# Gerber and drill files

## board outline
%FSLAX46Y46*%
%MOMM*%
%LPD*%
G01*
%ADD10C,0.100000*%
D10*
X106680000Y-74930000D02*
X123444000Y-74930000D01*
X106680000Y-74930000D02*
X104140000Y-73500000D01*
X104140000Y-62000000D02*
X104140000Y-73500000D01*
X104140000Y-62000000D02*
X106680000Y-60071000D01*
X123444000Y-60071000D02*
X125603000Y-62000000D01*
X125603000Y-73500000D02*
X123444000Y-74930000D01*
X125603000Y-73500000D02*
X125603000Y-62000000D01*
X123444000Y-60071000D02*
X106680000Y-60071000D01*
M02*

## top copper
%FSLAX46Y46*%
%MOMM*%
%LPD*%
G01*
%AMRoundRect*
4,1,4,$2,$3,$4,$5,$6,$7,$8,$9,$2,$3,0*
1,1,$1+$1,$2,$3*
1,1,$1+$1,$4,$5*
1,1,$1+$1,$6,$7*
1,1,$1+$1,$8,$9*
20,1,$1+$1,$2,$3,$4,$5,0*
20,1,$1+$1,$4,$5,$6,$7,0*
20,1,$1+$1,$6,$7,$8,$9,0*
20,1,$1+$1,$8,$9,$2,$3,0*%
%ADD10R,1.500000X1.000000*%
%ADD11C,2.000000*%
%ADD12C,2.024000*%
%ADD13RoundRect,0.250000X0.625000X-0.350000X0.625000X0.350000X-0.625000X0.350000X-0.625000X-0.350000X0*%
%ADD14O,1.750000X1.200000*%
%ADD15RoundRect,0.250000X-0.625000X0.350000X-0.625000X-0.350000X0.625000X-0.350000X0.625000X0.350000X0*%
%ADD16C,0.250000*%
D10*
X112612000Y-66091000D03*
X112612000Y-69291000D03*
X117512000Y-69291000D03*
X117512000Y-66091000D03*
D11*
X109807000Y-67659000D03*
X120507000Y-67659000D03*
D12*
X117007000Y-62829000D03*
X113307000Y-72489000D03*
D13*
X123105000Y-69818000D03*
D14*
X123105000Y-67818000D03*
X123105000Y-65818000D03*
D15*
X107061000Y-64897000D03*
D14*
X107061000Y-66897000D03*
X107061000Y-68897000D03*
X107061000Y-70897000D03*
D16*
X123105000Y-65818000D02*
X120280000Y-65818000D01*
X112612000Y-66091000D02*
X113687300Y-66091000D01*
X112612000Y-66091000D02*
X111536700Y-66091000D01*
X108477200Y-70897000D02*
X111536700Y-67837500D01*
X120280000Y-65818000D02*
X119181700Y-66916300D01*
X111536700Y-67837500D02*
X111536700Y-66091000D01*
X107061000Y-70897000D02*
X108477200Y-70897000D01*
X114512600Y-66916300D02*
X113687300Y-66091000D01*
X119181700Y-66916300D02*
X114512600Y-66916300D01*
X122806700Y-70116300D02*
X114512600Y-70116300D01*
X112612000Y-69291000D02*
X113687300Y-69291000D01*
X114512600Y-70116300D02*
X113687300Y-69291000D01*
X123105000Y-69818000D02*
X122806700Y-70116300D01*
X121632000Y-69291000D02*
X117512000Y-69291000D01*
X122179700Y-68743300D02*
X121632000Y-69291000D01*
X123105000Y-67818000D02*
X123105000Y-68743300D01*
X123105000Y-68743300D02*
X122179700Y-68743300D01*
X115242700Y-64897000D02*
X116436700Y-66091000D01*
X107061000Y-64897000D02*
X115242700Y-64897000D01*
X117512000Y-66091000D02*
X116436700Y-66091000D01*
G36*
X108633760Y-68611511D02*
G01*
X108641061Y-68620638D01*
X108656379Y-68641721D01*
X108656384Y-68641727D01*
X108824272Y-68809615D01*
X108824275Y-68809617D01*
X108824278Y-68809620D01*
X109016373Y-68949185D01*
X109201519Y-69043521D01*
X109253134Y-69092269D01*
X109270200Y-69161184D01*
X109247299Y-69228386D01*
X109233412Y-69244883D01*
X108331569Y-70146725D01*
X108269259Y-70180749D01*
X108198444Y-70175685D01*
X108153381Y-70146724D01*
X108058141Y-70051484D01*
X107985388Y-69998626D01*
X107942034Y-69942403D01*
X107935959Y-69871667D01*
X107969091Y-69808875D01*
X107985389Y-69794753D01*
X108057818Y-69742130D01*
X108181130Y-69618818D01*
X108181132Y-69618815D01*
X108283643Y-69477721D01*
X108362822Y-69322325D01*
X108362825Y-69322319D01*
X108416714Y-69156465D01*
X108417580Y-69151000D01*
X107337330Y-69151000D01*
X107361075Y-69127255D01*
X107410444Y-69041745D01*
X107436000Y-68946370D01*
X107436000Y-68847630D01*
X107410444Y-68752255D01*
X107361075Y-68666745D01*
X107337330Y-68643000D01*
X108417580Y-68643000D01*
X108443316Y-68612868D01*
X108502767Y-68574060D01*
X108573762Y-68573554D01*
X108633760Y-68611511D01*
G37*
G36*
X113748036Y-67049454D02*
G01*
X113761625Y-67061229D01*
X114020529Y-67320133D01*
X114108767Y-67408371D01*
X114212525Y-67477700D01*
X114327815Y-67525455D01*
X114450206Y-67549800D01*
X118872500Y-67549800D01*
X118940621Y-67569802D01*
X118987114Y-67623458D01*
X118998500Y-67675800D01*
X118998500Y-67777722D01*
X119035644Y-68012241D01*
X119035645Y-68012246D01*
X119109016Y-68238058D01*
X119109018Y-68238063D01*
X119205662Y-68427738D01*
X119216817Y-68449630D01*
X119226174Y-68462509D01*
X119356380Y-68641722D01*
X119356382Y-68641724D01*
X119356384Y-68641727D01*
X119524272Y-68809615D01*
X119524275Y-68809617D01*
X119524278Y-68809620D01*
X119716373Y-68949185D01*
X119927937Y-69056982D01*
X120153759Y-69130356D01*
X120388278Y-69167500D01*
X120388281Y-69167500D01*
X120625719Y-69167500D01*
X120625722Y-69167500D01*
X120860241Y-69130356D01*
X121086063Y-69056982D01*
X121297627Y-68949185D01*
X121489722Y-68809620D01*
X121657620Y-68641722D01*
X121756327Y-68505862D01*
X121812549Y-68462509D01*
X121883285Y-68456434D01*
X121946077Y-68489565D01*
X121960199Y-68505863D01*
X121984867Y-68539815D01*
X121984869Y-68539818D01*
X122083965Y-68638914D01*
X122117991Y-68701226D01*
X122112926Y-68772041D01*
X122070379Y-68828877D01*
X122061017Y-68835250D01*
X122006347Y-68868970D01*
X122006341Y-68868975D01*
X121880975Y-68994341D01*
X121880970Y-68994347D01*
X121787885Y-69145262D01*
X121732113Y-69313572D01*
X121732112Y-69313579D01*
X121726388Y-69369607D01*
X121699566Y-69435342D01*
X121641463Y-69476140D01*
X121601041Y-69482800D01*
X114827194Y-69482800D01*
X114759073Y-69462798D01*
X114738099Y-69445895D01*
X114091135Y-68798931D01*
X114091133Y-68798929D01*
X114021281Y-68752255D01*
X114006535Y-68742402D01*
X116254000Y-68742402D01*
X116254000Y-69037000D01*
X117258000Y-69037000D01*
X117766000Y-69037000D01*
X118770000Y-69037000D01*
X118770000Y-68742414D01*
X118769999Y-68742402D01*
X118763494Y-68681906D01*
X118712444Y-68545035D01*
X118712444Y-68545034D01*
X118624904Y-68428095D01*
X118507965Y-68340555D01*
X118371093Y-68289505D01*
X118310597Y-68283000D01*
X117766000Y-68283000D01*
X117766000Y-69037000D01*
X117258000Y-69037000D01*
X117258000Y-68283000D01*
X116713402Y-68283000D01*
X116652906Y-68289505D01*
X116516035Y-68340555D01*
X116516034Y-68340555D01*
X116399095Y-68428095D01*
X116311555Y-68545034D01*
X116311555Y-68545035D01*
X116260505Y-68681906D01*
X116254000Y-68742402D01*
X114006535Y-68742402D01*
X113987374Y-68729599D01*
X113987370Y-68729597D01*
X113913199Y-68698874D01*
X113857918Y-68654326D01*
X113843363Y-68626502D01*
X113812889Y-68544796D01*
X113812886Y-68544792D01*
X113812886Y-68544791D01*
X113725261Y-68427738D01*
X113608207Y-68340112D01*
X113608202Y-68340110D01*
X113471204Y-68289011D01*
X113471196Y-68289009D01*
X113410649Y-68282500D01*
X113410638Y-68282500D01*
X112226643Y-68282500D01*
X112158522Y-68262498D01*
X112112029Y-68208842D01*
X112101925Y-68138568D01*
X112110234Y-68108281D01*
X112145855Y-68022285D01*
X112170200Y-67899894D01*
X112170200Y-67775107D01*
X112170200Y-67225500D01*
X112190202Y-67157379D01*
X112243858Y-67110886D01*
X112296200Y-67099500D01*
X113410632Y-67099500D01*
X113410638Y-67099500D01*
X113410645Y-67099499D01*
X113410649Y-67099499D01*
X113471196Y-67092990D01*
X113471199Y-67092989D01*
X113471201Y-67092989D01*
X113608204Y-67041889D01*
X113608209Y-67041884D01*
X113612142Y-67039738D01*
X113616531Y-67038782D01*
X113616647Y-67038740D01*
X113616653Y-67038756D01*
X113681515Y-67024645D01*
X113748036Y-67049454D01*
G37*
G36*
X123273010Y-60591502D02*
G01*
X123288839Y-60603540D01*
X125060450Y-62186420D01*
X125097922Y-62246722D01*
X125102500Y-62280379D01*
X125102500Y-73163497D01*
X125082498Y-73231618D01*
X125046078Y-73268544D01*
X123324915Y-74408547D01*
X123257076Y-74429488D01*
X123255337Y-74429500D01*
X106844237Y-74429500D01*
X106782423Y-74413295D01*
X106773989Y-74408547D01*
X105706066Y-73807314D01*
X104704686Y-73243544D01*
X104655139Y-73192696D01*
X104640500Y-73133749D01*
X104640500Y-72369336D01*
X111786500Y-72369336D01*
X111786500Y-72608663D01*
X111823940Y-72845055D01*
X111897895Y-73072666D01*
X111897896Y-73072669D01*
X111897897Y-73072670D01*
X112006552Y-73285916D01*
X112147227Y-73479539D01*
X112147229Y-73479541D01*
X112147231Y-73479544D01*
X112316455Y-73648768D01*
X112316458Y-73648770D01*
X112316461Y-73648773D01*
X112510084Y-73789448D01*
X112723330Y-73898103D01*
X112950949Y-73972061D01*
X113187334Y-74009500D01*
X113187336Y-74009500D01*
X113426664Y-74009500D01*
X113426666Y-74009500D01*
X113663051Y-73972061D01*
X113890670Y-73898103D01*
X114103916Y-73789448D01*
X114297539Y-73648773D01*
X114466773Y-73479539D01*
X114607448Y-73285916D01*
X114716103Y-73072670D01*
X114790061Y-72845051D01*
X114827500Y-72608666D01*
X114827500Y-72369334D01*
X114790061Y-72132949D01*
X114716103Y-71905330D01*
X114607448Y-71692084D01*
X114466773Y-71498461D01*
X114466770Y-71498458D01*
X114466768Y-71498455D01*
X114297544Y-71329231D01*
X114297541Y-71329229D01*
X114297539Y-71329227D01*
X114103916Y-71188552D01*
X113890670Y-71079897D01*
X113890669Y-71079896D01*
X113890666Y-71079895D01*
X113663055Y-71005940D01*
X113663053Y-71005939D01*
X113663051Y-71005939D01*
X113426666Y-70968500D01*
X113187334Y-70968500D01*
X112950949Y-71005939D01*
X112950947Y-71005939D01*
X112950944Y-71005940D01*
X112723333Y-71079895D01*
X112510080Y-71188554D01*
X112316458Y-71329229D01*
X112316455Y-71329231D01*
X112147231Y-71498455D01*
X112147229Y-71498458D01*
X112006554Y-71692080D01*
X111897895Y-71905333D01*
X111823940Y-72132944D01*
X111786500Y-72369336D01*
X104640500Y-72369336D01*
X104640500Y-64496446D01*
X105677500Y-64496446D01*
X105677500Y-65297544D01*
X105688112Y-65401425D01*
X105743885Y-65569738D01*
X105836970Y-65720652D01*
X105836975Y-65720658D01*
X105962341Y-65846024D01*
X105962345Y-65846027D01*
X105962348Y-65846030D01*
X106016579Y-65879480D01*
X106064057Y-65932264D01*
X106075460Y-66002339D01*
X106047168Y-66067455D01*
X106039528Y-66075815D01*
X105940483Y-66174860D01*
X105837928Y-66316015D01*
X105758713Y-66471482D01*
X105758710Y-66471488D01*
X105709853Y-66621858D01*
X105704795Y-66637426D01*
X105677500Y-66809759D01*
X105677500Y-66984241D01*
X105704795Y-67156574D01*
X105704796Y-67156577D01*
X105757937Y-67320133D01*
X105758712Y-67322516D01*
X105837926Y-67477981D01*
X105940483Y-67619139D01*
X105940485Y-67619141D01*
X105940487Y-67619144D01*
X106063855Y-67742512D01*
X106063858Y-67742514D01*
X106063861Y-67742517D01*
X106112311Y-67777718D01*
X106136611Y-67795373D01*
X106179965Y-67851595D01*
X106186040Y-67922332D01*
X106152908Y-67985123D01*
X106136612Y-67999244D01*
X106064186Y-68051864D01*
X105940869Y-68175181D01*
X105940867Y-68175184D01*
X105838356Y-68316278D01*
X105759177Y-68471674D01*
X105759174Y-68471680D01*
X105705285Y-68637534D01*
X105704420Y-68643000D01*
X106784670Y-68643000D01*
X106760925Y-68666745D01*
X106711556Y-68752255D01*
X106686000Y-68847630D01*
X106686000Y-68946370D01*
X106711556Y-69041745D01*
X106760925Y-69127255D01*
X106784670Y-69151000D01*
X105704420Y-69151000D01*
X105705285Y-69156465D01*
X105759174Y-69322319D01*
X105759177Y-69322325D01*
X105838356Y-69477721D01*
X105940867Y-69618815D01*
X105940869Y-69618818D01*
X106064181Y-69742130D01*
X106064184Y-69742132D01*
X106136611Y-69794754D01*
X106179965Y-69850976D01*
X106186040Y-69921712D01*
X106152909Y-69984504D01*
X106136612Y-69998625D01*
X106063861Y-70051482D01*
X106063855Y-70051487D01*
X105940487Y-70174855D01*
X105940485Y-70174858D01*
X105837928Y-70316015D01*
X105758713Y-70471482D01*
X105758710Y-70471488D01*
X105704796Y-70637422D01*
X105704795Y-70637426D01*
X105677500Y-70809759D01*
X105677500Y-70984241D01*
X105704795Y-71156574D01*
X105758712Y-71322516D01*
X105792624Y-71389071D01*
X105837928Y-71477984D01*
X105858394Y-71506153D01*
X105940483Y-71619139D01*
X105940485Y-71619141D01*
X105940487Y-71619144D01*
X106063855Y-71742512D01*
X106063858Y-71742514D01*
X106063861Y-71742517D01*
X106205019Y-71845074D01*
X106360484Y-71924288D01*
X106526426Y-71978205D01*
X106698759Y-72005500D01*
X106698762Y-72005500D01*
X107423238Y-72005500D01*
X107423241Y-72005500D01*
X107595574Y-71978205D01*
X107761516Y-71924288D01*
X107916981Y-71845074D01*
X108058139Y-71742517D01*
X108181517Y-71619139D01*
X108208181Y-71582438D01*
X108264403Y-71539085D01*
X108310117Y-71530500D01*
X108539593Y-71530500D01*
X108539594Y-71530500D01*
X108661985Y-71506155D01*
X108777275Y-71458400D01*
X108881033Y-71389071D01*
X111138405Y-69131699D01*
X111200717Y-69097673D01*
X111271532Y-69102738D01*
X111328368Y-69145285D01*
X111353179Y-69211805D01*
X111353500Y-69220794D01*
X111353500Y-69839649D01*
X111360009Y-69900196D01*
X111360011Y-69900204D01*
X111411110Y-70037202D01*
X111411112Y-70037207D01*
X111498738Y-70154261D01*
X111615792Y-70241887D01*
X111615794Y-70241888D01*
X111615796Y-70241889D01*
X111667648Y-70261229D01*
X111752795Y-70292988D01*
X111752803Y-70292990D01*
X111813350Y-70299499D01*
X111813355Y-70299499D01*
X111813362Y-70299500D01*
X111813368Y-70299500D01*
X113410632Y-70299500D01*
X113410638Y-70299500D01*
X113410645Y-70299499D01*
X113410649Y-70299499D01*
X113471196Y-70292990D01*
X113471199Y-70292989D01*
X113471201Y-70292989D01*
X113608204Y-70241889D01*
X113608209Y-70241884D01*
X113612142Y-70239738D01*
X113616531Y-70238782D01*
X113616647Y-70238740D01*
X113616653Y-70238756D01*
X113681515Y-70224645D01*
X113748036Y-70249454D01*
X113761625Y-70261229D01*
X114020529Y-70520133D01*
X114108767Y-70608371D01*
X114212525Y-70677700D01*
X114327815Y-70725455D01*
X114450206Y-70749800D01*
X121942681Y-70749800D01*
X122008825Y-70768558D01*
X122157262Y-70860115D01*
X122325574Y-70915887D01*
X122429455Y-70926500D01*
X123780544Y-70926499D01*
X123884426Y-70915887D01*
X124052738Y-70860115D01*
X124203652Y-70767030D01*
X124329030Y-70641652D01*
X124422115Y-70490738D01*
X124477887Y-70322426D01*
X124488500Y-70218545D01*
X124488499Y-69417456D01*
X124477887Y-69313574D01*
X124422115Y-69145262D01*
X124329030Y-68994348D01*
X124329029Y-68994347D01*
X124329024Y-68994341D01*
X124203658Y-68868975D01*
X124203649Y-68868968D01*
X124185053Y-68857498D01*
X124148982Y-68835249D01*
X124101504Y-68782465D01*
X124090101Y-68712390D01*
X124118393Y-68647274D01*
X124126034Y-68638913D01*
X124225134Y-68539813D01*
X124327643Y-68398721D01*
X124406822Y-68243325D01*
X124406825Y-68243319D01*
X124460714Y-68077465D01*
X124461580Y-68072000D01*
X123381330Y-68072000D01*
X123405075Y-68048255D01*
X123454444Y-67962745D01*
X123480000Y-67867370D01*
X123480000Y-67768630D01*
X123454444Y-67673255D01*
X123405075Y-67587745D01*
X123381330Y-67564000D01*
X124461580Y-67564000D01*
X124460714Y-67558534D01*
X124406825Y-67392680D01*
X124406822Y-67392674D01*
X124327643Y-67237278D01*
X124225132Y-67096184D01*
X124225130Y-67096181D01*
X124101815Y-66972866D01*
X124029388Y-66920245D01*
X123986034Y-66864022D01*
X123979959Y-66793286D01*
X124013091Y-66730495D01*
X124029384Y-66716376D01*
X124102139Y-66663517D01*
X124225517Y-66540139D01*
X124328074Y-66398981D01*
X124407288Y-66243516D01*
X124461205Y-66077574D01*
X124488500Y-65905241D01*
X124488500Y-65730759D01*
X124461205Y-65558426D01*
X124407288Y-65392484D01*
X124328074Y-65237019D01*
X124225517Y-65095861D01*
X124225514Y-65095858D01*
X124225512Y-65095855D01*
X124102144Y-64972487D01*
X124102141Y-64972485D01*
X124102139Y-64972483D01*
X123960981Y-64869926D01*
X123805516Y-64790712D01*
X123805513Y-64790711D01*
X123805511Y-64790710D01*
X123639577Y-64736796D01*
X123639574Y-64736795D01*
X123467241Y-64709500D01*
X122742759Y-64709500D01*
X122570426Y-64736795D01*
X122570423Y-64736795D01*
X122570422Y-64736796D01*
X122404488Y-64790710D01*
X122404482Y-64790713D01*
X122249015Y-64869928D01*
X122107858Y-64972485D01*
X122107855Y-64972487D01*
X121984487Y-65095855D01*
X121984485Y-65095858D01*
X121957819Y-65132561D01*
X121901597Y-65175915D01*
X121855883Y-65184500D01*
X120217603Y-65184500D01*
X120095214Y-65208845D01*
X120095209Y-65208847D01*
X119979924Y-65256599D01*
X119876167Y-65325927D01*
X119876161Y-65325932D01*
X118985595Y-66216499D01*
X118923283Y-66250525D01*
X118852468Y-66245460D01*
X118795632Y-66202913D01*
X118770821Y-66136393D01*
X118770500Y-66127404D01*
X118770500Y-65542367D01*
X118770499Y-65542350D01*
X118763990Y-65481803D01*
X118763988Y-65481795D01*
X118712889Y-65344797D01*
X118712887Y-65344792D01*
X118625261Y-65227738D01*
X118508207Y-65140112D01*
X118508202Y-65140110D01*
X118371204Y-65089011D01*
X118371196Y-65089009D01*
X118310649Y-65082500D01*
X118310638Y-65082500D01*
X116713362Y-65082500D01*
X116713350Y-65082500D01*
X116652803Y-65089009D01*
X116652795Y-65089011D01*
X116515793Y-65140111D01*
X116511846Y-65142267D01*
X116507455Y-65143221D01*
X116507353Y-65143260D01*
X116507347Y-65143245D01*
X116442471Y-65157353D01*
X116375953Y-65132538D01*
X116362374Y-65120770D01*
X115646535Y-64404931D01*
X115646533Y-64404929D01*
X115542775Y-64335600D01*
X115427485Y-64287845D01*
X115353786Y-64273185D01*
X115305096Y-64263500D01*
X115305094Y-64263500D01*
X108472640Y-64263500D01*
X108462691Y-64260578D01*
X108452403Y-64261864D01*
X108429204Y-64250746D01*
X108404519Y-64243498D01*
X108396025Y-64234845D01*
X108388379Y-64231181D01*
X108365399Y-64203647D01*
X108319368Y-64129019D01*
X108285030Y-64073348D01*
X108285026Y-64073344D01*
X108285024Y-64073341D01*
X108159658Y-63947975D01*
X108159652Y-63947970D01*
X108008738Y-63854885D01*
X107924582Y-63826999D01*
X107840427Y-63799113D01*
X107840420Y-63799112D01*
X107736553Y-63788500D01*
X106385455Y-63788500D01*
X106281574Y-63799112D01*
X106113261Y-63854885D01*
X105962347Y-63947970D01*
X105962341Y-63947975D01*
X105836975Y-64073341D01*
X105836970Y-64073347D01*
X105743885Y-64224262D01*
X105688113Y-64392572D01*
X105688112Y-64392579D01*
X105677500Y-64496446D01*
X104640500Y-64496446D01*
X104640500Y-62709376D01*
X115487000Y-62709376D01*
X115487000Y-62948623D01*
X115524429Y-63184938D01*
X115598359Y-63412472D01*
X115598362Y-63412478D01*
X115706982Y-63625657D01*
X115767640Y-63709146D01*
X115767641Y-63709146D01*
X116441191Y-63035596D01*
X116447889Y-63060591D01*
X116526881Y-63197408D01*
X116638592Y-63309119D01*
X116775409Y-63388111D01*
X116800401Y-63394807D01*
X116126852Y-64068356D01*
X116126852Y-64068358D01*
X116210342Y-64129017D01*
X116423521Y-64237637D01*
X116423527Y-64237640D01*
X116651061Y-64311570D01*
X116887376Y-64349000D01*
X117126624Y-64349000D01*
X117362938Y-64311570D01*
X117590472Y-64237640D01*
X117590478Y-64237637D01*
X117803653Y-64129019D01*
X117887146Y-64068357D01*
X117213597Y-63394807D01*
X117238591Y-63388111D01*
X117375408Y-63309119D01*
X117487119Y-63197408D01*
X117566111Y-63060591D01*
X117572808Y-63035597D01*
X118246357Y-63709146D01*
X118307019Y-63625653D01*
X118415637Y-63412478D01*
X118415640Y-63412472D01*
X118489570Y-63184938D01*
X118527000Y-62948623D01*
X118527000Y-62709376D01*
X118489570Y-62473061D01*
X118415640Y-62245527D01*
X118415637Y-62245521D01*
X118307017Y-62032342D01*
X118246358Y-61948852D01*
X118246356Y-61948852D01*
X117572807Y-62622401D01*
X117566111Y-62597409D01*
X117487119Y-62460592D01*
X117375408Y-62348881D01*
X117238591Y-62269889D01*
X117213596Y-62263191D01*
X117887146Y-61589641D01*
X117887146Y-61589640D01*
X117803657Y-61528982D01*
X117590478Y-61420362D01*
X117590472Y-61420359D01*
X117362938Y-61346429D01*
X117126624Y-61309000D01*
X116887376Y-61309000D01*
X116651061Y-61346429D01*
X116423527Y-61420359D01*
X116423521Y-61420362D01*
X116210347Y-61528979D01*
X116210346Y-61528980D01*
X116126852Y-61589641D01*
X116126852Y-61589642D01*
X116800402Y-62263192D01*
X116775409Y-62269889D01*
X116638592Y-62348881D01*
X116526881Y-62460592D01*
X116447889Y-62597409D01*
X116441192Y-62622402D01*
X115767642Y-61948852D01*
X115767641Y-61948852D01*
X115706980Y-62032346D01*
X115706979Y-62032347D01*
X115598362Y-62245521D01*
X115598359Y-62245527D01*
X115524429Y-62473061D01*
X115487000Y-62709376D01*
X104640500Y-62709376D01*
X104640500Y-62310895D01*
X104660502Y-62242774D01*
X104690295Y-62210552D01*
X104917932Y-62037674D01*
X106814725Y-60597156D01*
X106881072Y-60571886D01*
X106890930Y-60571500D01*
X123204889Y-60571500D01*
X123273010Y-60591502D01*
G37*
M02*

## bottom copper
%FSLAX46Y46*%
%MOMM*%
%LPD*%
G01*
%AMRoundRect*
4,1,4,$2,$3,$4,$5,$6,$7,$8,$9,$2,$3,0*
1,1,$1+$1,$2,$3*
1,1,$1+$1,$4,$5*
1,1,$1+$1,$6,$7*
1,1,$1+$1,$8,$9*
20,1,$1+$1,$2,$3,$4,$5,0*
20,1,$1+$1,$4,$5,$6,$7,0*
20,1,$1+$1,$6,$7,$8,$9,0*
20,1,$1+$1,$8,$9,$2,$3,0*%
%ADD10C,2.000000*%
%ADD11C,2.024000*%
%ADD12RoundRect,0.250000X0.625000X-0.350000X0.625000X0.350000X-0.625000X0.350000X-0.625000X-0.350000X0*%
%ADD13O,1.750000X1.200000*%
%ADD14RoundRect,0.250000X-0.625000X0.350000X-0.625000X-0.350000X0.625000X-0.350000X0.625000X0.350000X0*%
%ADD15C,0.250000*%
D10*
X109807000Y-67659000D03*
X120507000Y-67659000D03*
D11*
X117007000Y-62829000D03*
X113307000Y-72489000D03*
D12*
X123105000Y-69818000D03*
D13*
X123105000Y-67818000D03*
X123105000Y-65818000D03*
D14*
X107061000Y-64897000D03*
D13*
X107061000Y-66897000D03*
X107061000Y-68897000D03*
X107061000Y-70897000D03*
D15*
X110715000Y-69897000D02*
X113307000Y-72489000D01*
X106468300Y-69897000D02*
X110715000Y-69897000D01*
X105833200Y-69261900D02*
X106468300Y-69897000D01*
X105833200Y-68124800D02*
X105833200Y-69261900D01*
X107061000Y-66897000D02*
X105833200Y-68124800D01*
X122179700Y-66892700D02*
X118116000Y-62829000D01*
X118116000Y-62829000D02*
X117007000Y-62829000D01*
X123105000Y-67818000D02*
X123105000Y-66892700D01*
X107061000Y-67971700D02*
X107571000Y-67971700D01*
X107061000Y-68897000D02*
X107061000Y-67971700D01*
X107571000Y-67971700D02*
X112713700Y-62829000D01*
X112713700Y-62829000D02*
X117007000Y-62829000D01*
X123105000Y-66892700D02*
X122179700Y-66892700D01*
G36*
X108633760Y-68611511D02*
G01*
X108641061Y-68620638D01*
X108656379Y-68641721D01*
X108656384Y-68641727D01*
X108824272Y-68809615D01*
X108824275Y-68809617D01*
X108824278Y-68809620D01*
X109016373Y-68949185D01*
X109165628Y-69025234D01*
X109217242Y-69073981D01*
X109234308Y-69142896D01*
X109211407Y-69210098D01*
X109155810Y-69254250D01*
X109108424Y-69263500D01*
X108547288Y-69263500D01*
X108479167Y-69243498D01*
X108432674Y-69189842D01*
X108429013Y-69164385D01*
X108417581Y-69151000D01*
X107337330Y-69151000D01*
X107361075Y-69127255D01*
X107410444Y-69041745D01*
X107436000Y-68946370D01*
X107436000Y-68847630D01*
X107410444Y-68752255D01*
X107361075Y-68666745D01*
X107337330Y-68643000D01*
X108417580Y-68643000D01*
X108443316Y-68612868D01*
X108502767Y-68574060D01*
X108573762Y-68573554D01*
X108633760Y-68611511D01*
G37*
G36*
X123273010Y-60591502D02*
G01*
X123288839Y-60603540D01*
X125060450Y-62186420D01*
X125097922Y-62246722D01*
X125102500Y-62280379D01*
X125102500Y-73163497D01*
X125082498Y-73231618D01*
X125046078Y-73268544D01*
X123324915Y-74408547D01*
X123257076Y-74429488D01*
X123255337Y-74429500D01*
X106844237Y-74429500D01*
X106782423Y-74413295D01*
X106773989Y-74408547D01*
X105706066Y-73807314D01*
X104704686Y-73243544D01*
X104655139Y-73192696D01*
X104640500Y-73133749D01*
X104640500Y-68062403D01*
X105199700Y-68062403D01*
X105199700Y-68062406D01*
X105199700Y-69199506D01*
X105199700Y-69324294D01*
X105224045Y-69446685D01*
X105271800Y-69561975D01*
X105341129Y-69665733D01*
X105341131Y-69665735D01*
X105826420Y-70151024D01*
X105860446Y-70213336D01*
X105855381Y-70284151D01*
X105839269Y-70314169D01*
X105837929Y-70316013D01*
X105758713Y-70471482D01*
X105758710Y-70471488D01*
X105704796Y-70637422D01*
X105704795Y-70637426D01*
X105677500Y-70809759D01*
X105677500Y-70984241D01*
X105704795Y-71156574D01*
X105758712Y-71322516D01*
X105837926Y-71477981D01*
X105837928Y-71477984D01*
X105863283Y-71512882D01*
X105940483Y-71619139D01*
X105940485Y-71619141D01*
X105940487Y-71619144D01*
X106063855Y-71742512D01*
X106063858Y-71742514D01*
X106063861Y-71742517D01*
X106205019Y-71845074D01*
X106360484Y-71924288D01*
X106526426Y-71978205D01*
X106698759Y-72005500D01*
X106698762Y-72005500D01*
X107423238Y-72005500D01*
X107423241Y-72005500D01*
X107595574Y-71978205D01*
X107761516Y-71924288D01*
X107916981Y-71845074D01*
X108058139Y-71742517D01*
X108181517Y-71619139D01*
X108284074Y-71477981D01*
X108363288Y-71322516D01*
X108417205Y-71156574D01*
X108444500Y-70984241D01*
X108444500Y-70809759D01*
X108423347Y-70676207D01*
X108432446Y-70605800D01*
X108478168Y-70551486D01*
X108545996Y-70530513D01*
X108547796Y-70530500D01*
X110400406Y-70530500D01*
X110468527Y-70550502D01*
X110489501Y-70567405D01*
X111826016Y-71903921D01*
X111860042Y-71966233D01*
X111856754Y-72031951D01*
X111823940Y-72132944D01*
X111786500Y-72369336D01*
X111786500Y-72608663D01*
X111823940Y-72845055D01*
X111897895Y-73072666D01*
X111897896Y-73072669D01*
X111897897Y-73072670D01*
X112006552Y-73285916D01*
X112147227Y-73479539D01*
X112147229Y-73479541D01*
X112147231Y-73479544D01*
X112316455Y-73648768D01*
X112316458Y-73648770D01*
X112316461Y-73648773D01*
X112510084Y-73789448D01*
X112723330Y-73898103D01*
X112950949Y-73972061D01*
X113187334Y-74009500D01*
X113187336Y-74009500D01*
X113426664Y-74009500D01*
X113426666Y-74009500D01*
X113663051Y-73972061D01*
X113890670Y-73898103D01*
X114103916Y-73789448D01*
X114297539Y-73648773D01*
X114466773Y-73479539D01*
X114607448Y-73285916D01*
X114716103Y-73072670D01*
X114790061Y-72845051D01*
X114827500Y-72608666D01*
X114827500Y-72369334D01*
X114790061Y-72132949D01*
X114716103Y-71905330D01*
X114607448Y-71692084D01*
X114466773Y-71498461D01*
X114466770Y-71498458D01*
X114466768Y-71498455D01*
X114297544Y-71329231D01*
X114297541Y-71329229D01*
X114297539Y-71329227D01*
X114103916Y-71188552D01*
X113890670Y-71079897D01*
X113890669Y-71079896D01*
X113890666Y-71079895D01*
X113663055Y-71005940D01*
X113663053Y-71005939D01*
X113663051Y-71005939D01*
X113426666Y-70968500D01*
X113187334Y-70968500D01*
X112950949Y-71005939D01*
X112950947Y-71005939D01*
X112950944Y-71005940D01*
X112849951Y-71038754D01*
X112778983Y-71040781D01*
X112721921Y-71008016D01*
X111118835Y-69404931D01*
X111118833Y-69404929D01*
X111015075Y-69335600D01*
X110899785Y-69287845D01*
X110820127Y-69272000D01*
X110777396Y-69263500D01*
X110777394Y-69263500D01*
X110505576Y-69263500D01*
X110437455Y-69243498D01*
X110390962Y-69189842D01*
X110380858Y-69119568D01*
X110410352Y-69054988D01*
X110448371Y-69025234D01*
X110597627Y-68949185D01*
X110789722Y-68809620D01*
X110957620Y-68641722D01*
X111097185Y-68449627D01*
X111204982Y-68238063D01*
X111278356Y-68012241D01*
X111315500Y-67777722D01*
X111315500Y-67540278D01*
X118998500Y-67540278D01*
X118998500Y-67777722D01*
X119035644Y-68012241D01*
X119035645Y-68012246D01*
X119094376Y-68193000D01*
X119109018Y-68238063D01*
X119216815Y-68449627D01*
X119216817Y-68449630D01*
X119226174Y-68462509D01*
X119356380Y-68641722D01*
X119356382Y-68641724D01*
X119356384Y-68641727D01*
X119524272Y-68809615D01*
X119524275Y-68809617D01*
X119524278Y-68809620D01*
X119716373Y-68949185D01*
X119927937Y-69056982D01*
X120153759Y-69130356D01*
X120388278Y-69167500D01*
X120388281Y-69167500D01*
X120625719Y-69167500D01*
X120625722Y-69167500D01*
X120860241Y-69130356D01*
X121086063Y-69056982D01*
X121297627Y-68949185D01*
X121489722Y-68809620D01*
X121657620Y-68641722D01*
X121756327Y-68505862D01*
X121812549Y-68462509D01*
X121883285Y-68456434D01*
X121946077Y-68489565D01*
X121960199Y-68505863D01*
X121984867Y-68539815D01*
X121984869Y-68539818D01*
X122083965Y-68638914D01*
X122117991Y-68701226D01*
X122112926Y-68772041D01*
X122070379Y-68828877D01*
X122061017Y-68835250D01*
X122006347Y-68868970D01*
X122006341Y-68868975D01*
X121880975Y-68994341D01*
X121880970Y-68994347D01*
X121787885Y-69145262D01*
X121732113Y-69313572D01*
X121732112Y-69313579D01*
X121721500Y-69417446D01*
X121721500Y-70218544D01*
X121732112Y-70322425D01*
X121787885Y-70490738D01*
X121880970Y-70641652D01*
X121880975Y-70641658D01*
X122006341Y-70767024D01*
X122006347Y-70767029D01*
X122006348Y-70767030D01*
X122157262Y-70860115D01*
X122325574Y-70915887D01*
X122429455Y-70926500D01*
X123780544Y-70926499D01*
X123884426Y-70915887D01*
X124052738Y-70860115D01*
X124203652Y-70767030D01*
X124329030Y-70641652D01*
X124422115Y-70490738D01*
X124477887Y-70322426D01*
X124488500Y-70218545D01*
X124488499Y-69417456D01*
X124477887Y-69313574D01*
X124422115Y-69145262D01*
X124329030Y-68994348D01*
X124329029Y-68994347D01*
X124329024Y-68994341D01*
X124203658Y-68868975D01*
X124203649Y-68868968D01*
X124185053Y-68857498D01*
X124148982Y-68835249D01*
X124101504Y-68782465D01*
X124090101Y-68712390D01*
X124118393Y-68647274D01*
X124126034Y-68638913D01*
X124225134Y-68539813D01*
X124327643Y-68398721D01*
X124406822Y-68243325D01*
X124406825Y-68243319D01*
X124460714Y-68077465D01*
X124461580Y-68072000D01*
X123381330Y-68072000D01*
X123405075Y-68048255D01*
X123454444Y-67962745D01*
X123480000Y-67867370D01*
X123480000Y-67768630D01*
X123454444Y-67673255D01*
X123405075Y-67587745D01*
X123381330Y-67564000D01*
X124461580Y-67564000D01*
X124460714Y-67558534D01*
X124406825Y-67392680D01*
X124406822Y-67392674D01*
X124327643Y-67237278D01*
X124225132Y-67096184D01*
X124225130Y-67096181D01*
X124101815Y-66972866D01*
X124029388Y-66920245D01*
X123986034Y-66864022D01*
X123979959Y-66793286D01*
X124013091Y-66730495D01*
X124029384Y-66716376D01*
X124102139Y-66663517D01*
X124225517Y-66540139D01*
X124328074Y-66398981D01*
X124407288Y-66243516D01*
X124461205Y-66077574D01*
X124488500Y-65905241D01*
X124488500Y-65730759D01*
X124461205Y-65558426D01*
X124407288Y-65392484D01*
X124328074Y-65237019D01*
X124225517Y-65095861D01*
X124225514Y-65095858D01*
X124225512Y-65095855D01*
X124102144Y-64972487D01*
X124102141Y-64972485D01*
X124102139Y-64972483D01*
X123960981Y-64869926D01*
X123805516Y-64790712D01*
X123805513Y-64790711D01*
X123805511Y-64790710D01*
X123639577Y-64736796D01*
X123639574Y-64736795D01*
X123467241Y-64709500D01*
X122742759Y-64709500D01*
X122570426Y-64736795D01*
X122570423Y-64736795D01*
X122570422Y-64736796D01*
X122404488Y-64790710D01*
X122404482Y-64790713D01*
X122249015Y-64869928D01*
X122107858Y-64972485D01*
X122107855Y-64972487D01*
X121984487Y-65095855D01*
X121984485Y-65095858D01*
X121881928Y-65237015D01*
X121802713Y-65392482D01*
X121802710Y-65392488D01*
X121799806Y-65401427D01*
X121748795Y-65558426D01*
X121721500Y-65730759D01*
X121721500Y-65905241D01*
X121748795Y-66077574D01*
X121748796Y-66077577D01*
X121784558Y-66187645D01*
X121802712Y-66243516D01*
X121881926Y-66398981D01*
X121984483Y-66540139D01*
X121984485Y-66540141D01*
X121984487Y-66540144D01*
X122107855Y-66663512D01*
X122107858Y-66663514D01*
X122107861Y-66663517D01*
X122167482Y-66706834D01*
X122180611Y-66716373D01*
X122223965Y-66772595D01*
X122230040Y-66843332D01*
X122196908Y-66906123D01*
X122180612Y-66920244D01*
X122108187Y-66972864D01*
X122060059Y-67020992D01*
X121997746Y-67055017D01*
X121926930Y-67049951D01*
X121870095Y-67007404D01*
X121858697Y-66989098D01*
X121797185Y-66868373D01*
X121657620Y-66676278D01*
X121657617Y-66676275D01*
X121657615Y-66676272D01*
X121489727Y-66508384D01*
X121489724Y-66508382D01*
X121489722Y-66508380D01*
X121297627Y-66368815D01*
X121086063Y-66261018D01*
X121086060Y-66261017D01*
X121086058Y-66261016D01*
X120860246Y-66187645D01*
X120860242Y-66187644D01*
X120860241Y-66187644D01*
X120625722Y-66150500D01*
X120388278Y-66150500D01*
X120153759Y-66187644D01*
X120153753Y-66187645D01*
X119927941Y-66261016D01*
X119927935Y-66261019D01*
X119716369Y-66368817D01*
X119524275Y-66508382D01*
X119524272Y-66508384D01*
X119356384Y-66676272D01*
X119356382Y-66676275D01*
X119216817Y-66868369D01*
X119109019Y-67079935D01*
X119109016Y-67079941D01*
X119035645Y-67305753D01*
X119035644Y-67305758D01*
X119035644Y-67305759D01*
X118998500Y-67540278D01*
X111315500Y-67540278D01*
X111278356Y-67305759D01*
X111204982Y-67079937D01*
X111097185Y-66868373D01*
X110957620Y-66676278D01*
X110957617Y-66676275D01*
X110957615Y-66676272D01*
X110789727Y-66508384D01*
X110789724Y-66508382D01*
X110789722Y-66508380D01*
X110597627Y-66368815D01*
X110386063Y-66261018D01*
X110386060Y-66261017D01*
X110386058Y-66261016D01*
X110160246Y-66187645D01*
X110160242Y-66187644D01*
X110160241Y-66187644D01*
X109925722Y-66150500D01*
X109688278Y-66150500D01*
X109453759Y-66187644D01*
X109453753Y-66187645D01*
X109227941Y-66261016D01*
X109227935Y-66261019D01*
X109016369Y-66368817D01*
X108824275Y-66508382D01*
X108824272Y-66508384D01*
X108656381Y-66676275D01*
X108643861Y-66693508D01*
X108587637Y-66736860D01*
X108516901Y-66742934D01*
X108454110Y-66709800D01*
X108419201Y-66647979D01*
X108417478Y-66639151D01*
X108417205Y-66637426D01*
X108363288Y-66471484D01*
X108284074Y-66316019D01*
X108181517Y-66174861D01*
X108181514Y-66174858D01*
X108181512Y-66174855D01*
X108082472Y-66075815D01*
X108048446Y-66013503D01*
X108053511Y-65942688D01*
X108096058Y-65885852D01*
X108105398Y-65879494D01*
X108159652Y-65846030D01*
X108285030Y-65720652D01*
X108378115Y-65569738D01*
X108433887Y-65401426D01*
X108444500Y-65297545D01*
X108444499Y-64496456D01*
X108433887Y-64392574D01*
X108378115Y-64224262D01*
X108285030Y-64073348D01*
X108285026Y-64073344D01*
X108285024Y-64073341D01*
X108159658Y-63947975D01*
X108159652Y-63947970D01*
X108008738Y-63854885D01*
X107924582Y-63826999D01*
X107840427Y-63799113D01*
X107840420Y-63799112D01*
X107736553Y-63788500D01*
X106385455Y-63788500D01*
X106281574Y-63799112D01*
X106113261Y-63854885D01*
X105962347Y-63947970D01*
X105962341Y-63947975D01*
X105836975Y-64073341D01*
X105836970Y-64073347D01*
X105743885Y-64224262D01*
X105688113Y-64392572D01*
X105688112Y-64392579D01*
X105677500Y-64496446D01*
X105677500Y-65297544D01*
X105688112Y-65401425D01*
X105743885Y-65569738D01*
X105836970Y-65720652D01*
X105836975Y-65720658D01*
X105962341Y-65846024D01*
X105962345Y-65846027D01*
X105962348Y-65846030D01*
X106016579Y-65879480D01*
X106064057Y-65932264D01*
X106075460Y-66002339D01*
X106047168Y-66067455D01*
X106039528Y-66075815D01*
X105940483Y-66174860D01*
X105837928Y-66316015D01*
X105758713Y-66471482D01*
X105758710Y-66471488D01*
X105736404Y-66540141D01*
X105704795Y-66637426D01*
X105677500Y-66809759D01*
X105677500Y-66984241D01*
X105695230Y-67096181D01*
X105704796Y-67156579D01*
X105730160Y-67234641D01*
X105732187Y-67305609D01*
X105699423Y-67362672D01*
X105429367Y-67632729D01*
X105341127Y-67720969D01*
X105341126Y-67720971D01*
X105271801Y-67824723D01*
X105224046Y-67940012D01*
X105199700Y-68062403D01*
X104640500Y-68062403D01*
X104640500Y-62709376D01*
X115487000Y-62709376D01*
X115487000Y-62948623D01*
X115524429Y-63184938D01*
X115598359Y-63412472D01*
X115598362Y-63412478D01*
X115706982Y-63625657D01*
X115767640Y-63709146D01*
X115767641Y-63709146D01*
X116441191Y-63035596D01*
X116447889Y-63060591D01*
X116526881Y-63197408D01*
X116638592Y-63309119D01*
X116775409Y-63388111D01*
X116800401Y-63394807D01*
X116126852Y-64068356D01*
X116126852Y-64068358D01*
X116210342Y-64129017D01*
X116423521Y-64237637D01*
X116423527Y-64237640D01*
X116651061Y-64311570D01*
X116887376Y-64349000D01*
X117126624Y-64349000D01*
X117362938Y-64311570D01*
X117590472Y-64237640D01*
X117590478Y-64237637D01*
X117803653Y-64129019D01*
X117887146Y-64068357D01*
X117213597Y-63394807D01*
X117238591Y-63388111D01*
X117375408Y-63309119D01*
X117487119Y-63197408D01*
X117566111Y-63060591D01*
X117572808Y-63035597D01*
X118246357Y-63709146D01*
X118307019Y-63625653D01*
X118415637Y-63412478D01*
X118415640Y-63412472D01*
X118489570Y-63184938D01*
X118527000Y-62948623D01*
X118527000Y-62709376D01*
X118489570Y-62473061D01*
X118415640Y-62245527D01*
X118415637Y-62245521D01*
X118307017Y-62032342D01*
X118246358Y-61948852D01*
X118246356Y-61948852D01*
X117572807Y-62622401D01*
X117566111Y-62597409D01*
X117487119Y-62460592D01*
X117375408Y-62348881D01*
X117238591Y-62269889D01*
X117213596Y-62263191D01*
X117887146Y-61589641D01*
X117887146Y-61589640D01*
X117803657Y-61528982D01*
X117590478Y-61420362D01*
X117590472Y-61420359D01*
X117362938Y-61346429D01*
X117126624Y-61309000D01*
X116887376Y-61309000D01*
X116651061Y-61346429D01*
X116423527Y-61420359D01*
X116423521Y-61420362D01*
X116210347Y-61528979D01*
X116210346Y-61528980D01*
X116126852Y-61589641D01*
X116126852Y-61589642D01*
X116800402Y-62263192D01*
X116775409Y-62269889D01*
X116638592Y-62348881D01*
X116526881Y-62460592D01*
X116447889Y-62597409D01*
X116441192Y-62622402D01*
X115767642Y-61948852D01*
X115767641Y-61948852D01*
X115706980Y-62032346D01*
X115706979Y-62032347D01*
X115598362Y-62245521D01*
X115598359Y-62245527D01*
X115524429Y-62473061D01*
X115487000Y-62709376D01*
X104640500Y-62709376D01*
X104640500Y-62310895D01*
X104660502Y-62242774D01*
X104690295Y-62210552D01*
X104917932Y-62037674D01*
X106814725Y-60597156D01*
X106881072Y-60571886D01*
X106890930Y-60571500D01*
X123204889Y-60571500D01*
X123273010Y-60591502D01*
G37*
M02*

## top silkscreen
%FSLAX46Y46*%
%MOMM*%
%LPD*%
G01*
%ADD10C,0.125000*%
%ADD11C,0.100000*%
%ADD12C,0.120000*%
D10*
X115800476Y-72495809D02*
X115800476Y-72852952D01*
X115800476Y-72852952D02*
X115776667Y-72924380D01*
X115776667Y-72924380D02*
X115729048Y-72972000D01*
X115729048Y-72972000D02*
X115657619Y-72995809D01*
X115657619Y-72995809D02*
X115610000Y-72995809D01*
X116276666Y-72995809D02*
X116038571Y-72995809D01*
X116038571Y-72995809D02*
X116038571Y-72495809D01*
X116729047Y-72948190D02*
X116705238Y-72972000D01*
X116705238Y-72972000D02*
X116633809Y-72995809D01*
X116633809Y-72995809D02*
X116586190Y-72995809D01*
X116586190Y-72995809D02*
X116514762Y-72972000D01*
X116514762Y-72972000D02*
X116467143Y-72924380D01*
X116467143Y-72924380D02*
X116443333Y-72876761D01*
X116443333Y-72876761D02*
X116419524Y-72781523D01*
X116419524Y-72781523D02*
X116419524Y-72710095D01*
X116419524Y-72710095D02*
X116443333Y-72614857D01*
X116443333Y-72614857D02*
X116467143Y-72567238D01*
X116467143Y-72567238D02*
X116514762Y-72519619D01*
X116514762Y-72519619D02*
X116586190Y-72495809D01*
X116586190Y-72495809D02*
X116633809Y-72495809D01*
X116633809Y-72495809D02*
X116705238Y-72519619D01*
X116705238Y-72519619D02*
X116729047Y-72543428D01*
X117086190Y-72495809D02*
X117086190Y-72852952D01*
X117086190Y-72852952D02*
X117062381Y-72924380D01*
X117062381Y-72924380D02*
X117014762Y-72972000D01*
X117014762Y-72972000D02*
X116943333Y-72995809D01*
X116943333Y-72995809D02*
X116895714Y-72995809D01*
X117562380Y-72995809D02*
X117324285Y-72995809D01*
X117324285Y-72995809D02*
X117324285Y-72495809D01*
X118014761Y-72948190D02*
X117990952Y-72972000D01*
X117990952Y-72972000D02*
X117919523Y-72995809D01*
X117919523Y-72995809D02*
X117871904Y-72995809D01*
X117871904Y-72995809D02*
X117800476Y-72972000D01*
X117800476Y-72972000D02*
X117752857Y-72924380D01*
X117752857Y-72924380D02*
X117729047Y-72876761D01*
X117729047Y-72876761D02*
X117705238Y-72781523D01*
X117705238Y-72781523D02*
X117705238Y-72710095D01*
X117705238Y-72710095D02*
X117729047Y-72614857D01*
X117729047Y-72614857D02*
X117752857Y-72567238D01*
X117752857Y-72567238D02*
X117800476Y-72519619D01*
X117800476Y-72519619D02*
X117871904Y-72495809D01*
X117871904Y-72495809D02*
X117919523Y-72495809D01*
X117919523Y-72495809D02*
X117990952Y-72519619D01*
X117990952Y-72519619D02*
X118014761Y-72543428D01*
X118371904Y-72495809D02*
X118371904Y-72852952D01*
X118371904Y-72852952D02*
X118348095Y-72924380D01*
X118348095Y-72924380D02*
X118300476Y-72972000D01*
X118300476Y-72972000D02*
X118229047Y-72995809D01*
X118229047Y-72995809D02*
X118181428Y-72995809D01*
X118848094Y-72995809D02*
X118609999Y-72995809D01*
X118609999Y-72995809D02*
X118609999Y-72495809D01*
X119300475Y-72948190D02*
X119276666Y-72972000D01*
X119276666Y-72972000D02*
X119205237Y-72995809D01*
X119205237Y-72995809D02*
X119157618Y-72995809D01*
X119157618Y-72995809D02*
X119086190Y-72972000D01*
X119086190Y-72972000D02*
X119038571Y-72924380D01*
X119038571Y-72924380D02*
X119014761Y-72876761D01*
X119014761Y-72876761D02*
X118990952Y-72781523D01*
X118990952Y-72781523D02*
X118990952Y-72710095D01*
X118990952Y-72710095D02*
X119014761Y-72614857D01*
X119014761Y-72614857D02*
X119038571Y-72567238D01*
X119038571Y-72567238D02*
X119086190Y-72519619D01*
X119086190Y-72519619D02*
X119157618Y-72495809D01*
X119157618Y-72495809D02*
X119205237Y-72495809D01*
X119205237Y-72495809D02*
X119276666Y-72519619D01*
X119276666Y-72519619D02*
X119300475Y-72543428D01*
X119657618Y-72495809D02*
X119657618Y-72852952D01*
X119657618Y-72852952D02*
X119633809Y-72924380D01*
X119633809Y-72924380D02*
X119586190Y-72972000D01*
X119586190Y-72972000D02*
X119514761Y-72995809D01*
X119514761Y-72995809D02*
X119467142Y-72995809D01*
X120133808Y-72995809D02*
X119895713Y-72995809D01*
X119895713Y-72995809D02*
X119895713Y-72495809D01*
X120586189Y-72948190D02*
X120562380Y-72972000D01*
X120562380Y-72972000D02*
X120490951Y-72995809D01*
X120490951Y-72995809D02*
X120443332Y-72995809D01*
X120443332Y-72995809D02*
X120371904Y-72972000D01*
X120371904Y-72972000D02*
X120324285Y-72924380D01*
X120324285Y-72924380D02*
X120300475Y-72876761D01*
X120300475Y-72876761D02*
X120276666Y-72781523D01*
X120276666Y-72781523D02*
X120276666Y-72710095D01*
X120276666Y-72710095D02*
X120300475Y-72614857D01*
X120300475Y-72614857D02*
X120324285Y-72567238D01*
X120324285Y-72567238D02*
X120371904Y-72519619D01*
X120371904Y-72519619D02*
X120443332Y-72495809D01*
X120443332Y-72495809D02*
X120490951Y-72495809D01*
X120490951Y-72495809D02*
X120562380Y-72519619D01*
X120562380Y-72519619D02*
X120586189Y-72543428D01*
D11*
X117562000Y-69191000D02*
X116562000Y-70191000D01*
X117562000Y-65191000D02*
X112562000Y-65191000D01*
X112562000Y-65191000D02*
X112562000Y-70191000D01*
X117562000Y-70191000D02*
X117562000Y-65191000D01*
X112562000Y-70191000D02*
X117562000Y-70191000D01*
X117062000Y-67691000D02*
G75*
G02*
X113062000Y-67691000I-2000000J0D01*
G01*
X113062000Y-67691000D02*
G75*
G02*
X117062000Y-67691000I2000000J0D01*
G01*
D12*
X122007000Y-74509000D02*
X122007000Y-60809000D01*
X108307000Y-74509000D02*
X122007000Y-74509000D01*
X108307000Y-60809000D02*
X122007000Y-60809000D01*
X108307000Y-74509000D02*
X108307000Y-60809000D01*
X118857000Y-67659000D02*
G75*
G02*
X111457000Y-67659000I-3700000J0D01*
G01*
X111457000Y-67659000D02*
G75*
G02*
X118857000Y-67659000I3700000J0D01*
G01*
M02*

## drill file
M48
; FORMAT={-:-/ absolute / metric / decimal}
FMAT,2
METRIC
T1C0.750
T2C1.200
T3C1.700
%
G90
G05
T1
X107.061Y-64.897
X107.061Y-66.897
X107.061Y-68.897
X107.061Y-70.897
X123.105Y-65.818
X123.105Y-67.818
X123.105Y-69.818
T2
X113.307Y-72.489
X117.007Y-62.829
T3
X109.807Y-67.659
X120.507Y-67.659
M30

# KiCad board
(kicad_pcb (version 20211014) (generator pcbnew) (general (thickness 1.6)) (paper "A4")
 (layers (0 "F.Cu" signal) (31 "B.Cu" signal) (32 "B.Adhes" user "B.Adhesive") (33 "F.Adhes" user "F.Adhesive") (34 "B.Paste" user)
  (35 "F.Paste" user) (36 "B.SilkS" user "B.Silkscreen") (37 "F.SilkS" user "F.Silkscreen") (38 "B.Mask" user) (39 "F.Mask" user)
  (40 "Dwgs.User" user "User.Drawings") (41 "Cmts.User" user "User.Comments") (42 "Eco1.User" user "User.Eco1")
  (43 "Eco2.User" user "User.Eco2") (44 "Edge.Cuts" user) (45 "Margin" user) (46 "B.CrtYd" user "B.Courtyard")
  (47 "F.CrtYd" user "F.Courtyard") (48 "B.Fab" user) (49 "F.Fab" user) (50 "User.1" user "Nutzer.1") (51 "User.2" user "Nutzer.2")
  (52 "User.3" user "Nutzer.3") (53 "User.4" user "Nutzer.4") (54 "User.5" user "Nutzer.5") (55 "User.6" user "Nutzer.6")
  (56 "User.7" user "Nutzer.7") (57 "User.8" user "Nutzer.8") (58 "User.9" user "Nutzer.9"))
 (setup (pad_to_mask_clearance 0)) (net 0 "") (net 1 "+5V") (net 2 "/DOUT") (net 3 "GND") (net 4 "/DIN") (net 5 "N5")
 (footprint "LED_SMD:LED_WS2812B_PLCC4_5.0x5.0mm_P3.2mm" (layer "F.Cu") (at 115.062 67.691)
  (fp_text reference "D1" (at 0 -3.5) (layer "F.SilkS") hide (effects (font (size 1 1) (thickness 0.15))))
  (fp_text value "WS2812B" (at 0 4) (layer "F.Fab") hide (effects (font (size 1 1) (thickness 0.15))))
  (fp_line (start 2.5 1.5) (end 1.5 2.5) (layer "F.SilkS") (width 0.1))
  (fp_line (start 2.5 -2.5) (end -2.5 -2.5) (layer "F.SilkS") (width 0.1))
  (fp_line (start -2.5 -2.5) (end -2.5 2.5) (layer "F.SilkS") (width 0.1))
  (fp_line (start 2.5 2.5) (end 2.5 -2.5) (layer "F.SilkS") (width 0.1))
  (fp_line (start -2.5 2.5) (end 2.5 2.5) (layer "F.SilkS") (width 0.1))
  (fp_circle (center 0 0) (end 2 0) (layer "F.SilkS") (width 0.1) (fill none))
  (pad "1" smd rect (at -2.45 -1.6) (size 1.5 1) (layers "F.Cu" "F.Paste" "F.Mask") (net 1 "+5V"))
  (pad "2" smd rect (at -2.45 1.6) (size 1.5 1) (layers "F.Cu" "F.Paste" "F.Mask") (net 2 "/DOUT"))
  (pad "3" smd rect (at 2.45 1.6) (size 1.5 1) (layers "F.Cu" "F.Paste" "F.Mask") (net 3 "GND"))
  (pad "4" smd rect (at 2.45 -1.6) (size 1.5 1) (layers "F.Cu" "F.Paste" "F.Mask") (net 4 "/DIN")))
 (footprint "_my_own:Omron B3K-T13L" (layer "F.Cu") (at 108.307 60.809)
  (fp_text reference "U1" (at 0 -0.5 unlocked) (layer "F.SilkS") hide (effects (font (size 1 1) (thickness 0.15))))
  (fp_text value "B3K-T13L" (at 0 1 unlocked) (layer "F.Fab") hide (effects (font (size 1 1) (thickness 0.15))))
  (fp_line (start 13.7 13.7) (end 13.7 0) (layer "F.SilkS") (width 0.12))
  (fp_line (start 0 13.7) (end 13.7 13.7) (layer "F.SilkS") (width 0.12))
  (fp_line (start 0 0) (end 13.7 0) (layer "F.SilkS") (width 0.12))
  (fp_line (start 0 13.7) (end 0 0) (layer "F.SilkS") (width 0.12))
  (fp_circle (center 6.85 6.85) (end 10.55 6.85) (layer "F.SilkS") (width 0.12) (fill none))
  (pad "" np_thru_hole circle (at 1.5 6.85) (size 2 2) (drill 1.7) (layers F&B.Cu *.Mask))
  (pad "" np_thru_hole circle (at 12.2 6.85) (size 2 2) (drill 1.7) (layers F&B.Cu *.Mask))
  (pad "1" thru_hole circle (at 8.7 2.02) (size 2.024 2.024) (drill 1.2) (layers *.Cu *.Mask) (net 3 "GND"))
  (pad "2" thru_hole circle (at 5 11.68) (size 2.024 2.024) (drill 1.2) (layers *.Cu *.Mask) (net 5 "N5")))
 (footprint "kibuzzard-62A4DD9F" (layer "B.Cu") (at 111.506 67.564 90)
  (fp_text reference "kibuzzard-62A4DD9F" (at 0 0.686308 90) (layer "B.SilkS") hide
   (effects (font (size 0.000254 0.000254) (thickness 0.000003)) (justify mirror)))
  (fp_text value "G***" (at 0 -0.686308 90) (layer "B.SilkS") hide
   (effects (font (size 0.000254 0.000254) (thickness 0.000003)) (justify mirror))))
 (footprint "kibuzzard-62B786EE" (layer "B.Cu") (at 118.618 67.945 -90)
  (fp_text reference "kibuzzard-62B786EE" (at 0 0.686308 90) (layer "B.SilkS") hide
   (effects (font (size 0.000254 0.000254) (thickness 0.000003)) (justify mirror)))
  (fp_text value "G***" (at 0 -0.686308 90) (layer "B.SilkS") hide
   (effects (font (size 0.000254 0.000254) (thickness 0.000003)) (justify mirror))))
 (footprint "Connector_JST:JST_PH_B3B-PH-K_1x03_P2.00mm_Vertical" (layer "B.Cu") (at 123.105 69.818 90)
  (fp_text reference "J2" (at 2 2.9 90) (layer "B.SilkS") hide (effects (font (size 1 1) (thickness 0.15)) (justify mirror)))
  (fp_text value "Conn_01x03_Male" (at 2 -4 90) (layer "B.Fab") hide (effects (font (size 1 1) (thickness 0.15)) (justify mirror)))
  (pad "1" thru_hole roundrect (at 0 0 90) (size 1.2 1.75) (drill 0.75) (layers *.Cu *.Mask) (roundrect_rratio 0.2083333333) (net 2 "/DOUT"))
  (pad "2" thru_hole oval (at 2 0 90) (size 1.2 1.75) (drill 0.75) (layers *.Cu *.Mask) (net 3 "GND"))
  (pad "3" thru_hole oval (at 4 0 90) (size 1.2 1.75) (drill 0.75) (layers *.Cu *.Mask) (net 1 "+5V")))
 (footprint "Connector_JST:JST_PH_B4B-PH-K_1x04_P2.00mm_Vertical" (layer "B.Cu") (at 107.061 64.897 -90)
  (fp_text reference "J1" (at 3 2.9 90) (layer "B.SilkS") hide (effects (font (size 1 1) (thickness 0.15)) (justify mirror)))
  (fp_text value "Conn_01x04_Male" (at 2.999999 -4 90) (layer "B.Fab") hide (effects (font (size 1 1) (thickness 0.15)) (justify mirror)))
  (pad "1" thru_hole roundrect (at 0 0 270) (size 1.2 1.75) (drill 0.75) (layers *.Cu *.Mask) (roundrect_rratio 0.2083333333) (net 4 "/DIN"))
  (pad "2" thru_hole oval (at 2 0 270) (size 1.2 1.75) (drill 0.75) (layers *.Cu *.Mask) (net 5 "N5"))
  (pad "3" thru_hole oval (at 4 0 270) (size 1.2 1.75) (drill 0.75) (layers *.Cu *.Mask) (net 3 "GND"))
  (pad "4" thru_hole oval (at 6 0 270) (size 1.2 1.75) (drill 0.75) (layers *.Cu *.Mask) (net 1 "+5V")))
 (gr_line (start 106.68 74.93) (end 123.444 74.93) (layer "Edge.Cuts") (width 0.1))
 (gr_line (start 106.68 74.93) (end 104.14 73.5) (layer "Edge.Cuts") (width 0.1))
 (gr_line (start 104.14 62) (end 104.14 73.5) (layer "Edge.Cuts") (width 0.1))
 (gr_line (start 104.14 62) (end 106.68 60.071) (layer "Edge.Cuts") (width 0.1))
 (gr_line (start 123.444 60.071) (end 125.603 62) (layer "Edge.Cuts") (width 0.1))
 (gr_line (start 125.603 73.5) (end 123.444 74.93) (layer "Edge.Cuts") (width 0.1))
 (gr_line (start 125.603 73.5) (end 125.603 62) (layer "Edge.Cuts") (width 0.1))
 (gr_line (start 123.444 60.071) (end 106.68 60.071) (layer "Edge.Cuts") (width 0.1))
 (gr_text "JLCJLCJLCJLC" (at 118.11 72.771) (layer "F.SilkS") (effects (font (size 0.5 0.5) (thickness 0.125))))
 (segment (start 123.105 65.818) (end 120.28 65.818) (width 0.25) (layer "F.Cu") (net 1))
 (segment (start 112.612 66.091) (end 113.6873 66.091) (width 0.25) (layer "F.Cu") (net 1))
 (segment (start 112.612 66.091) (end 111.5367 66.091) (width 0.25) (layer "F.Cu") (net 1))
 (segment (start 108.4772 70.897) (end 111.5367 67.8375) (width 0.25) (layer "F.Cu") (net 1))
 (segment (start 120.28 65.818) (end 119.1817 66.9163) (width 0.25) (layer "F.Cu") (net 1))
 (segment (start 111.5367 67.8375) (end 111.5367 66.091) (width 0.25) (layer "F.Cu") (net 1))
 (segment (start 107.061 70.897) (end 108.4772 70.897) (width 0.25) (layer "F.Cu") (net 1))
 (segment (start 114.5126 66.9163) (end 113.6873 66.091) (width 0.25) (layer "F.Cu") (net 1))
 (segment (start 119.1817 66.9163) (end 114.5126 66.9163) (width 0.25) (layer "F.Cu") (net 1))
 (segment (start 110.715 69.897) (end 113.307 72.489) (width 0.25) (layer "B.Cu") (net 5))
 (segment (start 106.4683 69.897) (end 110.715 69.897) (width 0.25) (layer "B.Cu") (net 5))
 (segment (start 105.8332 69.2619) (end 106.4683 69.897) (width 0.25) (layer "B.Cu") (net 5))
 (segment (start 105.8332 68.1248) (end 105.8332 69.2619) (width 0.25) (layer "B.Cu") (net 5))
 (segment (start 107.061 66.897) (end 105.8332 68.1248) (width 0.25) (layer "B.Cu") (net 5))
 (segment (start 122.8067 70.1163) (end 114.5126 70.1163) (width 0.25) (layer "F.Cu") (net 2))
 (segment (start 112.612 69.291) (end 113.6873 69.291) (width 0.25) (layer "F.Cu") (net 2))
 (segment (start 114.5126 70.1163) (end 113.6873 69.291) (width 0.25) (layer "F.Cu") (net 2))
 (segment (start 123.105 69.818) (end 122.8067 70.1163) (width 0.25) (layer "F.Cu") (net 2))
 (segment (start 121.632 69.291) (end 117.512 69.291) (width 0.25) (layer "F.Cu") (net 3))
 (segment (start 122.1797 68.7433) (end 121.632 69.291) (width 0.25) (layer "F.Cu") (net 3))
 (segment (start 123.105 67.818) (end 123.105 68.7433) (width 0.25) (layer "F.Cu") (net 3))
 (segment (start 123.105 68.7433) (end 122.1797 68.7433) (width 0.25) (layer "F.Cu") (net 3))
 (segment (start 122.1797 66.8927) (end 118.116 62.829) (width 0.25) (layer "B.Cu") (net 3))
 (segment (start 118.116 62.829) (end 117.007 62.829) (width 0.25) (layer "B.Cu") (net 3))
 (segment (start 123.105 67.818) (end 123.105 66.8927) (width 0.25) (layer "B.Cu") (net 3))
 (segment (start 107.061 67.9717) (end 107.571 67.9717) (width 0.25) (layer "B.Cu") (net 3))
 (segment (start 107.061 68.897) (end 107.061 67.9717) (width 0.25) (layer "B.Cu") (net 3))
 (segment (start 107.571 67.9717) (end 112.7137 62.829) (width 0.25) (layer "B.Cu") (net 3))
 (segment (start 112.7137 62.829) (end 117.007 62.829) (width 0.25) (layer "B.Cu") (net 3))
 (segment (start 123.105 66.8927) (end 122.1797 66.8927) (width 0.25) (layer "B.Cu") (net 3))
 (segment (start 115.2427 64.897) (end 116.4367 66.091) (width 0.25) (layer "F.Cu") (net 4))
 (segment (start 107.061 64.897) (end 115.2427 64.897) (width 0.25) (layer "F.Cu") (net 4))
 (segment (start 117.512 66.091) (end 116.4367 66.091) (width 0.25) (layer "F.Cu") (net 4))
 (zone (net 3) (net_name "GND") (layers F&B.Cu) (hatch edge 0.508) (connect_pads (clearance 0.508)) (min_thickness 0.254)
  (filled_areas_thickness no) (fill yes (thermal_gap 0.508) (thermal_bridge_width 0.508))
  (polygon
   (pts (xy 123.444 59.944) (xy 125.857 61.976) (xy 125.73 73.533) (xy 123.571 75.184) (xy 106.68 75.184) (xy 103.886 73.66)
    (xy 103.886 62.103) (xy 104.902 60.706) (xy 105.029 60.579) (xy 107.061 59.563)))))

